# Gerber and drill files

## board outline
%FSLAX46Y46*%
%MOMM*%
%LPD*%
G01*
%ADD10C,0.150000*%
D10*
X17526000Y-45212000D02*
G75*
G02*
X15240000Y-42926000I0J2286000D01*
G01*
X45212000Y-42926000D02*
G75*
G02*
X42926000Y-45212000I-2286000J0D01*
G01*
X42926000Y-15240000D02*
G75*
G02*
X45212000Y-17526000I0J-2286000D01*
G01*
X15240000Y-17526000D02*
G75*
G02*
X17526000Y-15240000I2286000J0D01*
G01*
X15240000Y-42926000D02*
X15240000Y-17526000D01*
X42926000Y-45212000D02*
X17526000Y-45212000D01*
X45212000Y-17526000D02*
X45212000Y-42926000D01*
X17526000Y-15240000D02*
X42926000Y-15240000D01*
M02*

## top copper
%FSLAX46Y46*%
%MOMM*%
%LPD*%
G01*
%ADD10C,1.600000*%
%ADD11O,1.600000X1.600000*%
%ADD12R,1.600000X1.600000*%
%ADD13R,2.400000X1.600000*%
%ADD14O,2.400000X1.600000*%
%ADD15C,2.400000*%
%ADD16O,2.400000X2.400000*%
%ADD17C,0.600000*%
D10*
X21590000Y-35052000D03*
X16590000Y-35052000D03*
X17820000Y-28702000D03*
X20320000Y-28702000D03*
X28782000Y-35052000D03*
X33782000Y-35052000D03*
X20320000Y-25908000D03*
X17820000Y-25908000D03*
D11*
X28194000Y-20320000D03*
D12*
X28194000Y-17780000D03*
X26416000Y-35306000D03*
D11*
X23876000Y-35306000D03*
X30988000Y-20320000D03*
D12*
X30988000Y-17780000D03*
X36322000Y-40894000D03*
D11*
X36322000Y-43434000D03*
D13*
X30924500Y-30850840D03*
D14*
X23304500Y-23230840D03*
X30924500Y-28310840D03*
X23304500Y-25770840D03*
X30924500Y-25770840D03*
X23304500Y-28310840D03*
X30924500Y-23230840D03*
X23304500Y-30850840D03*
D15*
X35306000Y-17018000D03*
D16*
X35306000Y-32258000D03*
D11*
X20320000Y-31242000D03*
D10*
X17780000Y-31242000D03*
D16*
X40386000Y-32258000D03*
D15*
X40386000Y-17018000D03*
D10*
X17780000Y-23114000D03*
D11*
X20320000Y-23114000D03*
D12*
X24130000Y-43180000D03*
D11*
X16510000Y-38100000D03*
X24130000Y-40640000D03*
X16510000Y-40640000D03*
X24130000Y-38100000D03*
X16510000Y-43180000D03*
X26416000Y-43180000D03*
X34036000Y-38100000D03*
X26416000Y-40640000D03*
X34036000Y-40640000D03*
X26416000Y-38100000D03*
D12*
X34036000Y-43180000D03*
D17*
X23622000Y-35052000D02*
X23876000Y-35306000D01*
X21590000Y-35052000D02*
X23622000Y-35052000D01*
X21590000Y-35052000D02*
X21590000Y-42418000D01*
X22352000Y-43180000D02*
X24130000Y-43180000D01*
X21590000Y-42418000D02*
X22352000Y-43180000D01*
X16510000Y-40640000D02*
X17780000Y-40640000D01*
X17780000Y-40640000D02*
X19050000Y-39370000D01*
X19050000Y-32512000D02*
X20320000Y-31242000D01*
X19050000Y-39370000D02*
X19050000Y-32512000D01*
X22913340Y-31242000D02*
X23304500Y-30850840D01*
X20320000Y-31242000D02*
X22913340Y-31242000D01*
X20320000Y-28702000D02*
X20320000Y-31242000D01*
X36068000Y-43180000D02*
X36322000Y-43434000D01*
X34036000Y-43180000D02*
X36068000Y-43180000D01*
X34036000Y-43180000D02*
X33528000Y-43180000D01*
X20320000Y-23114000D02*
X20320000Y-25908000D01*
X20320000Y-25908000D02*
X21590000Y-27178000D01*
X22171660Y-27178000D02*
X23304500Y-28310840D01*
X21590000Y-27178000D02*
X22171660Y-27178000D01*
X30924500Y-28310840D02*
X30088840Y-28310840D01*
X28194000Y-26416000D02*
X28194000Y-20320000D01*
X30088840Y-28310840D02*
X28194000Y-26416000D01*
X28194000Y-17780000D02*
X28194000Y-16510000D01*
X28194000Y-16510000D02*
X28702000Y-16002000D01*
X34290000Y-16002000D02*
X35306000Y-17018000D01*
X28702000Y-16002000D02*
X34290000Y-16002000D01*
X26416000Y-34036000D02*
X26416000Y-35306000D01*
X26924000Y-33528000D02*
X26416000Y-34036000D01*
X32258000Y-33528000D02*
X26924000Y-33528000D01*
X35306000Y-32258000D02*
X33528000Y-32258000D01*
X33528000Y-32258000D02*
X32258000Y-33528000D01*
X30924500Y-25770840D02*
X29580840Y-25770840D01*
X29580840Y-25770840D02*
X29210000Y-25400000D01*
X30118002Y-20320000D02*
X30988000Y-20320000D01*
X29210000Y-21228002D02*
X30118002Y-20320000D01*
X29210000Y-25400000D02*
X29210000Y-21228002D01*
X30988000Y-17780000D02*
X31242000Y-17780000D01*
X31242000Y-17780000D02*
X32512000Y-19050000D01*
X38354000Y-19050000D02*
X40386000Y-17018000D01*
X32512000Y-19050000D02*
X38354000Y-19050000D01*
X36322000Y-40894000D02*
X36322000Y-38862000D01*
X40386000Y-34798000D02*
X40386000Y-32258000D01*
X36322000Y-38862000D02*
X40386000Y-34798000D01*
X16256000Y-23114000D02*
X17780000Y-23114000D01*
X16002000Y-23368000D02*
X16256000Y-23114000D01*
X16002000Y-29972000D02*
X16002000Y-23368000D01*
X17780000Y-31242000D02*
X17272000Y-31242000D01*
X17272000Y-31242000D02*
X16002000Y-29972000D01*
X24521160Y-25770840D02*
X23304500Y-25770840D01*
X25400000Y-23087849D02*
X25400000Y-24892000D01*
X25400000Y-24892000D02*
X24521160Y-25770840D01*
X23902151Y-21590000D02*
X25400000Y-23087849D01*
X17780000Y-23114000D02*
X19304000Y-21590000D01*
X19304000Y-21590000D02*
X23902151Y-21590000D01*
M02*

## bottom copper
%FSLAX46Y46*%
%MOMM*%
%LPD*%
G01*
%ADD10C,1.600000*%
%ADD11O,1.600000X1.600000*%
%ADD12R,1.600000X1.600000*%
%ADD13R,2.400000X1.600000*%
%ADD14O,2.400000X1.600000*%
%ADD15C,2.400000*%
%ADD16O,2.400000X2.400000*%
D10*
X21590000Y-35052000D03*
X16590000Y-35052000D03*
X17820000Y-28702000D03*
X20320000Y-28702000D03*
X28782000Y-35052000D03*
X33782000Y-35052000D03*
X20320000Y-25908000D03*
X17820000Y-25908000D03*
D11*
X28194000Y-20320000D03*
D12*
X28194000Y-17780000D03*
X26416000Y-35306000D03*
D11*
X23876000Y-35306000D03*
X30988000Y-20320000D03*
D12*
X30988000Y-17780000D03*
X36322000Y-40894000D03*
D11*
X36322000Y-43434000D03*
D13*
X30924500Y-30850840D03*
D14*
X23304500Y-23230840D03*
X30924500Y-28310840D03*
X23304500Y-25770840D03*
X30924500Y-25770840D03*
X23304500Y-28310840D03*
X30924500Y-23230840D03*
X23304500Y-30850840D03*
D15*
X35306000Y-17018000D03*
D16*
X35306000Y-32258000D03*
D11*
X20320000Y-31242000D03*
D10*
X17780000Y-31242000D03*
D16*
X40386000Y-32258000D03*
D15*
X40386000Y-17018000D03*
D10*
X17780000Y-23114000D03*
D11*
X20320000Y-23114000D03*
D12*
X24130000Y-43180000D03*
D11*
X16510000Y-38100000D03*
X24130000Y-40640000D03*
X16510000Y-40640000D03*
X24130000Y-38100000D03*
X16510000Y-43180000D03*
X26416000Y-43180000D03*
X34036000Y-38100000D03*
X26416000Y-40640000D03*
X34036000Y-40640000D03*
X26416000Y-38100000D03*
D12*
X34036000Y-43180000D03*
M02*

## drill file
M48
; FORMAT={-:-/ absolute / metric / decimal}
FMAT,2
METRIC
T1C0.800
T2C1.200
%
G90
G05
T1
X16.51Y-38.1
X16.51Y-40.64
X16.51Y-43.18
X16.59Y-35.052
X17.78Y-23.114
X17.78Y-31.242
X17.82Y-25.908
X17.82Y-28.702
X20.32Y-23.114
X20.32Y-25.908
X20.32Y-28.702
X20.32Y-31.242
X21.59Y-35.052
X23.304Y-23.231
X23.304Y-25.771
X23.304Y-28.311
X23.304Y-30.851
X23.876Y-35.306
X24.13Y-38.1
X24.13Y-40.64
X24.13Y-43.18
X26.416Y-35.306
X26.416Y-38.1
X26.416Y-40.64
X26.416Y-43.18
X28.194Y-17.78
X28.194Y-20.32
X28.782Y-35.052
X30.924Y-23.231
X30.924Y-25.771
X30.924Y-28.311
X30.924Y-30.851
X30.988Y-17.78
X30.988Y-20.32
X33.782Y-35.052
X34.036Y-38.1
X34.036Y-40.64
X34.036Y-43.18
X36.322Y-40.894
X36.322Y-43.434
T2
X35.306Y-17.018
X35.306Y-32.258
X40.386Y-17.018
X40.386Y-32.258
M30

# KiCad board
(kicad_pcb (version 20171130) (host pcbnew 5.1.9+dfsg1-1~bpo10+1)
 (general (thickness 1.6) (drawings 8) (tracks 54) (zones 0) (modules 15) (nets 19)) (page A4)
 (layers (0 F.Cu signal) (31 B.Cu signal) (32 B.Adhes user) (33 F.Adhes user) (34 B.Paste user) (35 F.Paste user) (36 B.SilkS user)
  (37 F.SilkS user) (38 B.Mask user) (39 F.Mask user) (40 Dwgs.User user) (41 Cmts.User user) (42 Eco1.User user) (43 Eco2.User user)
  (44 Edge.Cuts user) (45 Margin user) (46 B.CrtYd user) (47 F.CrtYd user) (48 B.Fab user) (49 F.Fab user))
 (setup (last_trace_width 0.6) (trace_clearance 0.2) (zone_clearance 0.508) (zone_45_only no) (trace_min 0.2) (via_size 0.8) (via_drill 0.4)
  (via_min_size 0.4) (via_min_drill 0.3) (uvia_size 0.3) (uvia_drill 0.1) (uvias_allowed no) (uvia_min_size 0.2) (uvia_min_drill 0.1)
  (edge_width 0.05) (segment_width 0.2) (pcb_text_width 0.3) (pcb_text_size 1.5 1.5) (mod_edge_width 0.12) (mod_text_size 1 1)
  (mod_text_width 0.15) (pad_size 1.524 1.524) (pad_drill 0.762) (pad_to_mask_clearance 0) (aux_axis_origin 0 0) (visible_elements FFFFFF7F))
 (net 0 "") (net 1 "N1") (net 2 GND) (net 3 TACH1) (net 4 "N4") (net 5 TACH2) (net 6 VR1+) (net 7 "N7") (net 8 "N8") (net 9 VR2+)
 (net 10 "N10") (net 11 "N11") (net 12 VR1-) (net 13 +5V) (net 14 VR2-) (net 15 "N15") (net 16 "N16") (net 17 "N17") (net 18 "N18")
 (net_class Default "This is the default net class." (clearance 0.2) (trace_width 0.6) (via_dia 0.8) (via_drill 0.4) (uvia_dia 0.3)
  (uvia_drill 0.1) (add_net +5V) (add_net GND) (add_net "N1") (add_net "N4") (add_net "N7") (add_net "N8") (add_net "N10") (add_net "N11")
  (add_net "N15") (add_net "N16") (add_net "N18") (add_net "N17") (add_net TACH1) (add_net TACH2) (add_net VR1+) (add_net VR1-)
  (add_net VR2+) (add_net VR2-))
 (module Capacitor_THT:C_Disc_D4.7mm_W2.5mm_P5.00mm (layer F.Cu) (at 21.59 35.052 180)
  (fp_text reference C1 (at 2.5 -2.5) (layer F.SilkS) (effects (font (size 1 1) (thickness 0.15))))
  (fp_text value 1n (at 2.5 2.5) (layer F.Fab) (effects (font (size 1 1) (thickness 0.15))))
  (pad 1 thru_hole circle (at 0 0 180) (size 1.6 1.6) (drill 0.8) (layers *.Cu *.Mask) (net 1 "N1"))
  (pad 2 thru_hole circle (at 5 0 180) (size 1.6 1.6) (drill 0.8) (layers *.Cu *.Mask) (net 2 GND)))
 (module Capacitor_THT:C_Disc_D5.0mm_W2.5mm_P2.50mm (layer F.Cu) (at 20.32 28.702 180)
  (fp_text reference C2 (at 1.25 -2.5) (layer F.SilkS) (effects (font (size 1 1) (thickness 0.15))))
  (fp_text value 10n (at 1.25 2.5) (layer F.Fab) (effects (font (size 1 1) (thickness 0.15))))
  (pad 2 thru_hole circle (at 2.5 0 180) (size 1.6 1.6) (drill 0.8) (layers *.Cu *.Mask) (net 2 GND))
  (pad 1 thru_hole circle (at 0 0 180) (size 1.6 1.6) (drill 0.8) (layers *.Cu *.Mask) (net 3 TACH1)))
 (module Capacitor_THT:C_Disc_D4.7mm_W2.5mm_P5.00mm (layer F.Cu) (at 33.782 35.052 180)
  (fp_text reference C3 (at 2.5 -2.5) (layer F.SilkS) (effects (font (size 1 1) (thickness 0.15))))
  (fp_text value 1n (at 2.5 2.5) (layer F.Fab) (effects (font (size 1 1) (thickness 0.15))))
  (pad 2 thru_hole circle (at 5 0 180) (size 1.6 1.6) (drill 0.8) (layers *.Cu *.Mask) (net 2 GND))
  (pad 1 thru_hole circle (at 0 0 180) (size 1.6 1.6) (drill 0.8) (layers *.Cu *.Mask) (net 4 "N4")))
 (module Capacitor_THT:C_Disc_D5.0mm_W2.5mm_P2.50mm (layer F.Cu) (at 20.32 25.908 180)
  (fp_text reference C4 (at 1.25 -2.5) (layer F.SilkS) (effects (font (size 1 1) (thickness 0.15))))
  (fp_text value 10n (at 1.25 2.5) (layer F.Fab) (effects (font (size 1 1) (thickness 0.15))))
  (pad 1 thru_hole circle (at 0 0 180) (size 1.6 1.6) (drill 0.8) (layers *.Cu *.Mask) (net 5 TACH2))
  (pad 2 thru_hole circle (at 2.5 0 180) (size 1.6 1.6) (drill 0.8) (layers *.Cu *.Mask) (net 2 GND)))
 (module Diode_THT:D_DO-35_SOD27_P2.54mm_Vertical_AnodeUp (layer F.Cu) (at 28.194 17.78 270)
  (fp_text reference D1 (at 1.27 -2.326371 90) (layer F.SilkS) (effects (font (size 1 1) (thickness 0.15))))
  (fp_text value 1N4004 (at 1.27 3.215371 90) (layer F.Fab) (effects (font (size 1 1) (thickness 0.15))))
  (pad 2 thru_hole oval (at 2.54 0 270) (size 1.6 1.6) (drill 0.8) (layers *.Cu *.Mask) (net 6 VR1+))
  (pad 1 thru_hole rect (at 0 0 270) (size 1.6 1.6) (drill 0.8) (layers *.Cu *.Mask) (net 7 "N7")))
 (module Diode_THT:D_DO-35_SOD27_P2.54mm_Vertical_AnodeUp (layer F.Cu) (at 26.416 35.306 180)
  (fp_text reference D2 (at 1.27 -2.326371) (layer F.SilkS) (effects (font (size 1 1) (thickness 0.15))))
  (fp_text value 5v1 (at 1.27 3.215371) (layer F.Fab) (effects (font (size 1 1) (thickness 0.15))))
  (pad 1 thru_hole rect (at 0 0 180) (size 1.6 1.6) (drill 0.8) (layers *.Cu *.Mask) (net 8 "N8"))
  (pad 2 thru_hole oval (at 2.54 0 180) (size 1.6 1.6) (drill 0.8) (layers *.Cu *.Mask) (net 1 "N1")))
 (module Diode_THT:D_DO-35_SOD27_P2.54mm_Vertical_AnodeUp (layer F.Cu) (at 30.988 17.78 270)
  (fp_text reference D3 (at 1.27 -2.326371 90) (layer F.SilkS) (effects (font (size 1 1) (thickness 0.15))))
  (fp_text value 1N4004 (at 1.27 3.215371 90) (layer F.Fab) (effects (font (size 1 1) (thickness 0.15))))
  (pad 2 thru_hole oval (at 2.54 0 270) (size 1.6 1.6) (drill 0.8) (layers *.Cu *.Mask) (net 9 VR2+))
  (pad 1 thru_hole rect (at 0 0 270) (size 1.6 1.6) (drill 0.8) (layers *.Cu *.Mask) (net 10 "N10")))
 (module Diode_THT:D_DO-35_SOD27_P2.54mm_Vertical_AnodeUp (layer F.Cu) (at 36.322 40.894 270)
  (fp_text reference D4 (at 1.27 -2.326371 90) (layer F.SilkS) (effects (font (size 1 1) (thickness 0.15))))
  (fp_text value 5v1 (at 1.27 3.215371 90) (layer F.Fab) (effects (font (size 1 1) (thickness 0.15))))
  (pad 1 thru_hole rect (at 0 0 270) (size 1.6 1.6) (drill 0.8) (layers *.Cu *.Mask) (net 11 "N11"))
  (pad 2 thru_hole oval (at 2.54 0 270) (size 1.6 1.6) (drill 0.8) (layers *.Cu *.Mask) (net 4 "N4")))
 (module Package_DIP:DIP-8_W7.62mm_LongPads (layer F.Cu) (at 30.9245 30.85084 180)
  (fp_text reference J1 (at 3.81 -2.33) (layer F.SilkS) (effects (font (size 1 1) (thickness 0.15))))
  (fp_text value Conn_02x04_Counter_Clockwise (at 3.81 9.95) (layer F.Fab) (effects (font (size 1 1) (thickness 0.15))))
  (pad 1 thru_hole rect (at 0 0 180) (size 2.4 1.6) (drill 0.8) (layers *.Cu *.Mask) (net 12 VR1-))
  (pad 5 thru_hole oval (at 7.62 7.62 180) (size 2.4 1.6) (drill 0.8) (layers *.Cu *.Mask) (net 2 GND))
  (pad 2 thru_hole oval (at 0 2.54 180) (size 2.4 1.6) (drill 0.8) (layers *.Cu *.Mask) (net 6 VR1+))
  (pad 6 thru_hole oval (at 7.62 5.08 180) (size 2.4 1.6) (drill 0.8) (layers *.Cu *.Mask) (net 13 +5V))
  (pad 3 thru_hole oval (at 0 5.08 180) (size 2.4 1.6) (drill 0.8) (layers *.Cu *.Mask) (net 9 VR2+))
  (pad 7 thru_hole oval (at 7.62 2.54 180) (size 2.4 1.6) (drill 0.8) (layers *.Cu *.Mask) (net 5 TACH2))
  (pad 4 thru_hole oval (at 0 7.62 180) (size 2.4 1.6) (drill 0.8) (layers *.Cu *.Mask) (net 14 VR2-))
  (pad 8 thru_hole oval (at 7.62 0 180) (size 2.4 1.6) (drill 0.8) (layers *.Cu *.Mask) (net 3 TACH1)))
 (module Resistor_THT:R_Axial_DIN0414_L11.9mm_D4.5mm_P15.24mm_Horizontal (layer F.Cu) (at 35.306 17.018 270)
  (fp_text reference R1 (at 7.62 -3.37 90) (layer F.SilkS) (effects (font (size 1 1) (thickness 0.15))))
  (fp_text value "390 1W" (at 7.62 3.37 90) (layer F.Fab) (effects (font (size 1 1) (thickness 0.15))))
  (pad 1 thru_hole circle (at 0 0 270) (size 2.4 2.4) (drill 1.2) (layers *.Cu *.Mask) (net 7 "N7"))
  (pad 2 thru_hole oval (at 15.24 0 270) (size 2.4 2.4) (drill 1.2) (layers *.Cu *.Mask) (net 8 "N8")))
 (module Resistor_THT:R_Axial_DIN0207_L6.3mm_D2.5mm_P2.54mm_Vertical (layer F.Cu) (at 17.78 31.242)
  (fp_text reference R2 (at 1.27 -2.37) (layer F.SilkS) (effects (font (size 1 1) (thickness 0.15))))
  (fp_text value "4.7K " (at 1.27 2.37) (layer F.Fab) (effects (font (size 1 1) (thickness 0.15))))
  (pad 2 thru_hole oval (at 2.54 0) (size 1.6 1.6) (drill 0.8) (layers *.Cu *.Mask) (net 3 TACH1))
  (pad 1 thru_hole circle (at 0 0) (size 1.6 1.6) (drill 0.8) (layers *.Cu *.Mask) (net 13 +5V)))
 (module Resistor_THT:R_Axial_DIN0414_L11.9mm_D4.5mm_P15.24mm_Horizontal (layer F.Cu) (at 40.386 17.018 270)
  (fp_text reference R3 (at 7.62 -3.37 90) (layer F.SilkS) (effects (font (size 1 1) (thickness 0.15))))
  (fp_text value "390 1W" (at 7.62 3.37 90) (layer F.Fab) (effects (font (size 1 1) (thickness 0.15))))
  (pad 2 thru_hole oval (at 15.24 0 270) (size 2.4 2.4) (drill 1.2) (layers *.Cu *.Mask) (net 11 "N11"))
  (pad 1 thru_hole circle (at 0 0 270) (size 2.4 2.4) (drill 1.2) (layers *.Cu *.Mask) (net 10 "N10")))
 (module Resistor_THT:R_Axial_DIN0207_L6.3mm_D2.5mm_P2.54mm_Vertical (layer F.Cu) (at 17.78 23.114)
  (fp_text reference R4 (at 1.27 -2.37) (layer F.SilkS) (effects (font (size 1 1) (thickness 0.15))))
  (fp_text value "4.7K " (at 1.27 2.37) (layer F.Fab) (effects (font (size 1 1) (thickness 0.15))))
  (pad 1 thru_hole circle (at 0 0) (size 1.6 1.6) (drill 0.8) (layers *.Cu *.Mask) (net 13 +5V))
  (pad 2 thru_hole oval (at 2.54 0) (size 1.6 1.6) (drill 0.8) (layers *.Cu *.Mask) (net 5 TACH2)))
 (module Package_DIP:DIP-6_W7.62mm (layer F.Cu) (at 24.13 43.18 180)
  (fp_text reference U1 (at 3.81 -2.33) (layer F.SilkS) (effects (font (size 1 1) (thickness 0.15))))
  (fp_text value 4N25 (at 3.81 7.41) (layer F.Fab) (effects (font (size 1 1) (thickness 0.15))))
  (pad 1 thru_hole rect (at 0 0 180) (size 1.6 1.6) (drill 0.8) (layers *.Cu *.Mask) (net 1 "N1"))
  (pad 4 thru_hole oval (at 7.62 5.08 180) (size 1.6 1.6) (drill 0.8) (layers *.Cu *.Mask) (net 2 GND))
  (pad 2 thru_hole oval (at 0 2.54 180) (size 1.6 1.6) (drill 0.8) (layers *.Cu *.Mask) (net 2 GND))
  (pad 5 thru_hole oval (at 7.62 2.54 180) (size 1.6 1.6) (drill 0.8) (layers *.Cu *.Mask) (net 3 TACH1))
  (pad 3 thru_hole oval (at 0 5.08 180) (size 1.6 1.6) (drill 0.8) (layers *.Cu *.Mask) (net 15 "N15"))
  (pad 6 thru_hole oval (at 7.62 0 180) (size 1.6 1.6) (drill 0.8) (layers *.Cu *.Mask) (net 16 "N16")))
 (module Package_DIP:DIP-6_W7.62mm (layer F.Cu) (at 34.036 43.18 180)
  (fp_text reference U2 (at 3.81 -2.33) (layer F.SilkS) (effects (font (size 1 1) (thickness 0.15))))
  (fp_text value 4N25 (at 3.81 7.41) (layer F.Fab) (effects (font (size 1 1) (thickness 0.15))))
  (pad 6 thru_hole oval (at 7.62 0 180) (size 1.6 1.6) (drill 0.8) (layers *.Cu *.Mask) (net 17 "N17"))
  (pad 3 thru_hole oval (at 0 5.08 180) (size 1.6 1.6) (drill 0.8) (layers *.Cu *.Mask) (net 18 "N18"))
  (pad 5 thru_hole oval (at 7.62 2.54 180) (size 1.6 1.6) (drill 0.8) (layers *.Cu *.Mask) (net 5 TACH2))
  (pad 2 thru_hole oval (at 0 2.54 180) (size 1.6 1.6) (drill 0.8) (layers *.Cu *.Mask) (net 2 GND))
  (pad 4 thru_hole oval (at 7.62 5.08 180) (size 1.6 1.6) (drill 0.8) (layers *.Cu *.Mask) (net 2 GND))
  (pad 1 thru_hole rect (at 0 0 180) (size 1.6 1.6) (drill 0.8) (layers *.Cu *.Mask) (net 4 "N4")))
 (gr_arc (start 17.526 42.926) (end 15.24 42.926) (angle -90) (layer Edge.Cuts) (width 0.15))
 (gr_arc (start 42.926 42.926) (end 42.926 45.212) (angle -90) (layer Edge.Cuts) (width 0.15))
 (gr_arc (start 42.926 17.526) (end 45.212 17.526) (angle -90) (layer Edge.Cuts) (width 0.15))
 (gr_arc (start 17.526 17.526) (end 17.526 15.24) (angle -90) (layer Edge.Cuts) (width 0.15))
 (gr_line (start 15.24 42.926) (end 15.24 17.526) (layer Edge.Cuts) (width 0.15))
 (gr_line (start 42.926 45.212) (end 17.526 45.212) (layer Edge.Cuts) (width 0.15))
 (gr_line (start 45.212 17.526) (end 45.212 42.926) (layer Edge.Cuts) (width 0.15))
 (gr_line (start 17.526 15.24) (end 42.926 15.24) (layer Edge.Cuts) (width 0.15))
 (segment (start 23.622 35.052) (end 23.876 35.306) (width 0.6) (layer F.Cu) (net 1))
 (segment (start 21.59 35.052) (end 23.622 35.052) (width 0.6) (layer F.Cu) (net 1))
 (segment (start 21.59 35.052) (end 21.59 42.418) (width 0.6) (layer F.Cu) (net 1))
 (segment (start 22.352 43.18) (end 24.13 43.18) (width 0.6) (layer F.Cu) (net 1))
 (segment (start 21.59 42.418) (end 22.352 43.18) (width 0.6) (layer F.Cu) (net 1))
 (segment (start 16.51 40.64) (end 17.78 40.64) (width 0.6) (layer F.Cu) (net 3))
 (segment (start 17.78 40.64) (end 19.05 39.37) (width 0.6) (layer F.Cu) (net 3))
 (segment (start 19.05 32.512) (end 20.32 31.242) (width 0.6) (layer F.Cu) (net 3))
 (segment (start 19.05 39.37) (end 19.05 32.512) (width 0.6) (layer F.Cu) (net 3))
 (segment (start 22.91334 31.242) (end 23.3045 30.85084) (width 0.6) (layer F.Cu) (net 3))
 (segment (start 20.32 31.242) (end 22.91334 31.242) (width 0.6) (layer F.Cu) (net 3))
 (segment (start 20.32 28.702) (end 20.32 31.242) (width 0.6) (layer F.Cu) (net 3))
 (segment (start 36.068 43.18) (end 36.322 43.434) (width 0.6) (layer F.Cu) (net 4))
 (segment (start 34.036 43.18) (end 36.068 43.18) (width 0.6) (layer F.Cu) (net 4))
 (segment (start 34.036 43.18) (end 33.528 43.18) (width 0.6) (layer F.Cu) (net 4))
 (segment (start 20.32 23.114) (end 20.32 25.908) (width 0.6) (layer F.Cu) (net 5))
 (segment (start 20.32 25.908) (end 21.59 27.178) (width 0.6) (layer F.Cu) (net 5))
 (segment (start 22.17166 27.178) (end 23.3045 28.31084) (width 0.6) (layer F.Cu) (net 5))
 (segment (start 21.59 27.178) (end 22.17166 27.178) (width 0.6) (layer F.Cu) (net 5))
 (segment (start 30.9245 28.31084) (end 30.08884 28.31084) (width 0.6) (layer F.Cu) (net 6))
 (segment (start 28.194 26.416) (end 28.194 20.32) (width 0.6) (layer F.Cu) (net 6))
 (segment (start 30.08884 28.31084) (end 28.194 26.416) (width 0.6) (layer F.Cu) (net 6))
 (segment (start 28.194 17.78) (end 28.194 16.51) (width 0.6) (layer F.Cu) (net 7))
 (segment (start 28.194 16.51) (end 28.702 16.002) (width 0.6) (layer F.Cu) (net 7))
 (segment (start 34.29 16.002) (end 35.306 17.018) (width 0.6) (layer F.Cu) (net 7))
 (segment (start 28.702 16.002) (end 34.29 16.002) (width 0.6) (layer F.Cu) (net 7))
 (segment (start 26.416 34.036) (end 26.416 35.306) (width 0.6) (layer F.Cu) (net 8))
 (segment (start 26.924 33.528) (end 26.416 34.036) (width 0.6) (layer F.Cu) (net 8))
 (segment (start 32.258 33.528) (end 26.924 33.528) (width 0.6) (layer F.Cu) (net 8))
 (segment (start 35.306 32.258) (end 33.528 32.258) (width 0.6) (layer F.Cu) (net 8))
 (segment (start 33.528 32.258) (end 32.258 33.528) (width 0.6) (layer F.Cu) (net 8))
 (segment (start 30.9245 25.77084) (end 29.58084 25.77084) (width 0.6) (layer F.Cu) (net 9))
 (segment (start 29.58084 25.77084) (end 29.21 25.4) (width 0.6) (layer F.Cu) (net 9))
 (segment (start 30.118002 20.32) (end 30.988 20.32) (width 0.6) (layer F.Cu) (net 9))
 (segment (start 29.21 21.228002) (end 30.118002 20.32) (width 0.6) (layer F.Cu) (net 9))
 (segment (start 29.21 25.4) (end 29.21 21.228002) (width 0.6) (layer F.Cu) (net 9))
 (segment (start 30.988 17.78) (end 31.242 17.78) (width 0.6) (layer F.Cu) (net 10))
 (segment (start 31.242 17.78) (end 32.512 19.05) (width 0.6) (layer F.Cu) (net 10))
 (segment (start 38.354 19.05) (end 40.386 17.018) (width 0.6) (layer F.Cu) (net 10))
 (segment (start 32.512 19.05) (end 38.354 19.05) (width 0.6) (layer F.Cu) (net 10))
 (segment (start 36.322 40.894) (end 36.322 38.862) (width 0.6) (layer F.Cu) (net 11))
 (segment (start 40.386 34.798) (end 40.386 32.258) (width 0.6) (layer F.Cu) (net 11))
 (segment (start 36.322 38.862) (end 40.386 34.798) (width 0.6) (layer F.Cu) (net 11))
 (segment (start 16.256 23.114) (end 17.78 23.114) (width 0.6) (layer F.Cu) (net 13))
 (segment (start 16.002 23.368) (end 16.256 23.114) (width 0.6) (layer F.Cu) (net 13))
 (segment (start 16.002 29.972) (end 16.002 23.368) (width 0.6) (layer F.Cu) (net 13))
 (segment (start 17.78 31.242) (end 17.272 31.242) (width 0.6) (layer F.Cu) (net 13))
 (segment (start 17.272 31.242) (end 16.002 29.972) (width 0.6) (layer F.Cu) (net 13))
 (segment (start 24.52116 25.77084) (end 23.3045 25.77084) (width 0.6) (layer F.Cu) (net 13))
 (segment (start 25.4 23.087849) (end 25.4 24.892) (width 0.6) (layer F.Cu) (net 13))
 (segment (start 25.4 24.892) (end 24.52116 25.77084) (width 0.6) (layer F.Cu) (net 13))
 (segment (start 23.902151 21.59) (end 25.4 23.087849) (width 0.6) (layer F.Cu) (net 13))
 (segment (start 17.78 23.114) (end 19.304 21.59) (width 0.6) (layer F.Cu) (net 13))
 (segment (start 19.304 21.59) (end 23.902151 21.59) (width 0.6) (layer F.Cu) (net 13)))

